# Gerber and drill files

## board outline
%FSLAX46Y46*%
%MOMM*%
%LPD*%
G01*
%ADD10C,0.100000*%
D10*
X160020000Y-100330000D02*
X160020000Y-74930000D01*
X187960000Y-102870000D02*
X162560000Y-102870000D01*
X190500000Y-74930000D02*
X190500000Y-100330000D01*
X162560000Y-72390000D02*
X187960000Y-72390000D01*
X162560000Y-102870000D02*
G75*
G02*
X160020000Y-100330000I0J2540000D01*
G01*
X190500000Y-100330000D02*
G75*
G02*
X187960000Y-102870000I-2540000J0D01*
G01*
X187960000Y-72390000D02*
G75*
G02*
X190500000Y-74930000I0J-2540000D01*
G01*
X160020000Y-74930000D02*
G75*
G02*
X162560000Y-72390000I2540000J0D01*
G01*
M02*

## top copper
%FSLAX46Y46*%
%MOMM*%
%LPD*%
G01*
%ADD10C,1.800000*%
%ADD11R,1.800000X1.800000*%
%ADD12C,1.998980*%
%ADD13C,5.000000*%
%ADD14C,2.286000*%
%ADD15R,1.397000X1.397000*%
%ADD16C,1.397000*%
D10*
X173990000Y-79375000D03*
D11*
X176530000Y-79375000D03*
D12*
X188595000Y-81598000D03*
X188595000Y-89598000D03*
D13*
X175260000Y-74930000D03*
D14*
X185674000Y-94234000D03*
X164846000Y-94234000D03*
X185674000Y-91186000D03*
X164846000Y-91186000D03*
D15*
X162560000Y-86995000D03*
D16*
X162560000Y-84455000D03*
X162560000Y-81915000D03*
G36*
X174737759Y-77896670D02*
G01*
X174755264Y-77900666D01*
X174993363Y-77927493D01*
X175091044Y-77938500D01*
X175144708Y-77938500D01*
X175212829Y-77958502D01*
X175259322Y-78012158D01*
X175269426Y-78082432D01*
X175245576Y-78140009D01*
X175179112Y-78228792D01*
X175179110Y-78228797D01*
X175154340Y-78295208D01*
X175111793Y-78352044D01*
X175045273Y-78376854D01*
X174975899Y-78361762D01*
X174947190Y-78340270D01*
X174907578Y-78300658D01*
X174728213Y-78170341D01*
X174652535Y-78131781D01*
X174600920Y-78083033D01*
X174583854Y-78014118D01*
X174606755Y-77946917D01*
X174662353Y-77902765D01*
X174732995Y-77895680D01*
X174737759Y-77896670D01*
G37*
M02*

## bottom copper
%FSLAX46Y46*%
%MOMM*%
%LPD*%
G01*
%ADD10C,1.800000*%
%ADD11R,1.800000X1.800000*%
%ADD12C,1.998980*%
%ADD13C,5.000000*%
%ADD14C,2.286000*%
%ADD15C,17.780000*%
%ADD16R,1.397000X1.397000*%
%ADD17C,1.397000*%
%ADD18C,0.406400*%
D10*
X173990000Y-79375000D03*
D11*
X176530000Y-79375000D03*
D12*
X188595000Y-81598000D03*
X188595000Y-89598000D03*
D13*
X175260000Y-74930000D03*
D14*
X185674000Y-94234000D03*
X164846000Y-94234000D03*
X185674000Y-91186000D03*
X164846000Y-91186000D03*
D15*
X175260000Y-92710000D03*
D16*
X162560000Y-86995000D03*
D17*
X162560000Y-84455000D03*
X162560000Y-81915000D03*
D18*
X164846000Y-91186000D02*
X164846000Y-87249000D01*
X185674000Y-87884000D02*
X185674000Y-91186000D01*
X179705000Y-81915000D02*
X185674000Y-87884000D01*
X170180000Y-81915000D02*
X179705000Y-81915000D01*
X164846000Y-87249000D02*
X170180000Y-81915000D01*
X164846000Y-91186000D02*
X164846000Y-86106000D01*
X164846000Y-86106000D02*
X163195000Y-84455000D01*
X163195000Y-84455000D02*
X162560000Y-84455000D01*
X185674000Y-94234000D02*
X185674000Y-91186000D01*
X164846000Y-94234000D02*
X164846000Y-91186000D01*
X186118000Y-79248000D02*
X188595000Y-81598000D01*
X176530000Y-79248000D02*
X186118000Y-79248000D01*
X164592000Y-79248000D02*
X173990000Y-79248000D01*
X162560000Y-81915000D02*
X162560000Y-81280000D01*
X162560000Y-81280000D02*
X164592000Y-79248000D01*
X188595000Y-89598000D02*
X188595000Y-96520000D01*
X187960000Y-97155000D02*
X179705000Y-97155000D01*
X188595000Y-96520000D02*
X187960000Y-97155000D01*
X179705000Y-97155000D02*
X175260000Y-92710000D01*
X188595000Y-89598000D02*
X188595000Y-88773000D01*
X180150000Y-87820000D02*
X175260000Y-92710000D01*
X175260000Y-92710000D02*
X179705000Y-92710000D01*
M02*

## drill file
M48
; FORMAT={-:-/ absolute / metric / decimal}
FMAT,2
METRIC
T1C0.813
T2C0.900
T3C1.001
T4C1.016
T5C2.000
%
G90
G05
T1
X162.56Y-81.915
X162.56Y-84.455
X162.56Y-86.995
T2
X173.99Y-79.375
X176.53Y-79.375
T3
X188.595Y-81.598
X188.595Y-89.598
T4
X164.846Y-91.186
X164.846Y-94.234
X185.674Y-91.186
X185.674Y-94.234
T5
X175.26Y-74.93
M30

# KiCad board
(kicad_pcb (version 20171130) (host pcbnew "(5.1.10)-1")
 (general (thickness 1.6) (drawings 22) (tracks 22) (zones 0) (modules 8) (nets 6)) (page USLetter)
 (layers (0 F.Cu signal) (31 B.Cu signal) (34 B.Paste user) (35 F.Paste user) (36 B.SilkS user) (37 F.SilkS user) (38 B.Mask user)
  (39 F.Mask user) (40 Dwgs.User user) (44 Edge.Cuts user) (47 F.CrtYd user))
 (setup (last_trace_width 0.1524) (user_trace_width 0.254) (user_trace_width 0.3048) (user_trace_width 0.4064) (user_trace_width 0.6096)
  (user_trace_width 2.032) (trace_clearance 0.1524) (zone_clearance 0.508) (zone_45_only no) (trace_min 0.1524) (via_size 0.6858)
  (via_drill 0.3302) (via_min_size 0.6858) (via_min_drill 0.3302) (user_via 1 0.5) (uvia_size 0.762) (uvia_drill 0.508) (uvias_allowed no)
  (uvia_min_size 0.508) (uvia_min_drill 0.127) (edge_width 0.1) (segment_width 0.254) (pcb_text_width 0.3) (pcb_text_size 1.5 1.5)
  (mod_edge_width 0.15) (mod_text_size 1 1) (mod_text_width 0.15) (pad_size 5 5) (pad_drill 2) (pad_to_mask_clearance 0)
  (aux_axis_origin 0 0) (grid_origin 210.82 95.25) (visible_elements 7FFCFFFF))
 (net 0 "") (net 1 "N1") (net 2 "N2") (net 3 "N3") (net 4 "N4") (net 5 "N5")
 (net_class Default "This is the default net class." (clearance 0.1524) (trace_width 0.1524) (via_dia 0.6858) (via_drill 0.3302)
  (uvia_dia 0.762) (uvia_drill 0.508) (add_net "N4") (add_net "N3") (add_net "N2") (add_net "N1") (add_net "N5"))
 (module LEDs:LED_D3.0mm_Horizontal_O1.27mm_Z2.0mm (layer F.Cu) (at 173.99 79.375)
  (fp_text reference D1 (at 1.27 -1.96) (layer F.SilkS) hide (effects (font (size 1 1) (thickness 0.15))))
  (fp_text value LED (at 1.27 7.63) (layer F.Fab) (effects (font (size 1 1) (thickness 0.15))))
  (pad 2 thru_hole circle (at 0 0) (size 1.8 1.8) (drill 0.9) (layers *.Cu *.Mask) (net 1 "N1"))
  (pad 1 thru_hole rect (at 2.54 0) (size 1.8 1.8) (drill 0.9) (layers *.Cu *.Mask) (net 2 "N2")))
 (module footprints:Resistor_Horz (layer F.Cu) (at 188.595 85.598 270)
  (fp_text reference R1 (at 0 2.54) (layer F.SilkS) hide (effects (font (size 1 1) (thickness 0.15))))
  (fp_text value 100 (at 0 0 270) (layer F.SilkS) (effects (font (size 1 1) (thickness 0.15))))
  (pad 1 thru_hole circle (at -4 0 270) (size 1.99898 1.99898) (drill 1.00076) (layers *.Cu *.SilkS *.Mask) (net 2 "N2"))
  (pad 2 thru_hole circle (at 4 0 270) (size 1.99898 1.99898) (drill 1.00076) (layers *.Cu *.SilkS *.Mask) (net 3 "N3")))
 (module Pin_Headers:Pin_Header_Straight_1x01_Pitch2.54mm (layer F.Cu) (at 175.26 74.93)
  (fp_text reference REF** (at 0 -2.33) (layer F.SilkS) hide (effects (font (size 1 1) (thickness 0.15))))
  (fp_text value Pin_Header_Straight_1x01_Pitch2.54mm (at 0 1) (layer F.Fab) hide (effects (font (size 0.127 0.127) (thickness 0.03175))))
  (pad 1 thru_hole circle (at 0 0) (size 5 5) (drill 2) (layers *.Cu *.Mask)))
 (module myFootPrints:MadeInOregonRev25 (layer F.Cu) (at 167.64 76.454)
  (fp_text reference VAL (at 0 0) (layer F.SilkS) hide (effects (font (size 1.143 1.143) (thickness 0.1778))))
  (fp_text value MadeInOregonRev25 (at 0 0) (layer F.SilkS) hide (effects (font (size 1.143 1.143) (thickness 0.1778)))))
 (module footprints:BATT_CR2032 (layer B.Cu) (at 175.26 92.71 180)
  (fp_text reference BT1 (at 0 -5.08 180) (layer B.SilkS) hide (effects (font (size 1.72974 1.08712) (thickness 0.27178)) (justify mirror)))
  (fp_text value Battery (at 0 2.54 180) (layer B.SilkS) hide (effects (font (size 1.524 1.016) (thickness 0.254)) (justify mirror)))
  (pad 1 thru_hole circle (at -10.414 -1.524 180) (size 2.286 2.286) (drill 1.016) (layers *.Cu *.Mask B.SilkS) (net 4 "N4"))
  (pad 1 thru_hole circle (at 10.414 -1.524 180) (size 2.286 2.286) (drill 1.016) (layers *.Cu *.Mask B.SilkS) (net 4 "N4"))
  (pad 1 thru_hole circle (at -10.414 1.524 180) (size 2.286 2.286) (drill 1.016) (layers *.Cu *.Mask B.SilkS) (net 4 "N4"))
  (pad 1 thru_hole circle (at 10.414 1.524 180) (size 2.286 2.286) (drill 1.016) (layers *.Cu *.Mask B.SilkS) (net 4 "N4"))
  (pad 2 smd circle (at 0 0 180) (size 17.78 17.78) (layers B.Cu B.Paste B.Mask) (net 3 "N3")))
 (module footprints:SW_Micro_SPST (layer F.Cu) (at 162.56 84.455 90)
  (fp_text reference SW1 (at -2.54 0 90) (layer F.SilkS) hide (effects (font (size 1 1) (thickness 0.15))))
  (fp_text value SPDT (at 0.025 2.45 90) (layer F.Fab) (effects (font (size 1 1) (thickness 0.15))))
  (pad 1 thru_hole rect (at -2.54 0 90) (size 1.397 1.397) (drill 0.8128) (layers *.Cu *.Mask F.SilkS) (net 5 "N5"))
  (pad 2 thru_hole circle (at 0 0 90) (size 1.397 1.397) (drill 0.8128) (layers *.Cu *.Mask F.SilkS) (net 4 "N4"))
  (pad 3 thru_hole circle (at 2.54 0 90) (size 1.397 1.397) (drill 0.8128) (layers *.Cu *.Mask F.SilkS) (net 1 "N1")))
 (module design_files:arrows (layer F.Cu) (at 177.546 81.788)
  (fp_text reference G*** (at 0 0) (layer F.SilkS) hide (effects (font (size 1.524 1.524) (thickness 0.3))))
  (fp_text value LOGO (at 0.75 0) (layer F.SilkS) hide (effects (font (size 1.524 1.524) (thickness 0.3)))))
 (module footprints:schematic (layer F.Cu) (at 175.26 87.503)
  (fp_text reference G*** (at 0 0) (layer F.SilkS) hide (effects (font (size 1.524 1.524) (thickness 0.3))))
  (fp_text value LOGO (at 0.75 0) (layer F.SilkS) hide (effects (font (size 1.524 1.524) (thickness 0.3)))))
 (gr_line (start 160.02 100.33) (end 160.02 74.93) (angle 90) (layer Edge.Cuts) (width 0.1))
 (gr_line (start 187.96 102.87) (end 162.56 102.87) (angle 90) (layer Edge.Cuts) (width 0.1))
 (gr_line (start 190.5 74.93) (end 190.5 100.33) (angle 90) (layer Edge.Cuts) (width 0.1))
 (gr_line (start 162.56 72.39) (end 187.96 72.39) (angle 90) (layer Edge.Cuts) (width 0.1))
 (gr_arc (start 162.56 100.33) (end 162.56 102.87) (angle 90) (layer Edge.Cuts) (width 0.1))
 (gr_arc (start 187.96 100.33) (end 190.5 100.33) (angle 90) (layer Edge.Cuts) (width 0.1))
 (gr_arc (start 187.96 74.93) (end 187.96 72.39) (angle 90) (layer Edge.Cuts) (width 0.1))
 (gr_arc (start 162.56 74.93) (end 160.02 74.93) (angle 90) (layer Edge.Cuts) (width 0.1))
 (segment (start 164.846 91.186) (end 164.846 87.249) (width 0.4064) (layer B.Cu) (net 4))
 (segment (start 185.674 87.884) (end 185.674 91.186) (width 0.4064) (layer B.Cu) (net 4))
 (segment (start 179.705 81.915) (end 185.674 87.884) (width 0.4064) (layer B.Cu) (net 4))
 (segment (start 170.18 81.915) (end 179.705 81.915) (width 0.4064) (layer B.Cu) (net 4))
 (segment (start 164.846 87.249) (end 170.18 81.915) (width 0.4064) (layer B.Cu) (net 4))
 (segment (start 164.846 91.186) (end 164.846 86.106) (width 0.4064) (layer B.Cu) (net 4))
 (segment (start 164.846 86.106) (end 163.195 84.455) (width 0.4064) (layer B.Cu) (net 4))
 (segment (start 163.195 84.455) (end 162.56 84.455) (width 0.4064) (layer B.Cu) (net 4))
 (segment (start 185.674 94.234) (end 185.674 91.186) (width 0.4064) (layer B.Cu) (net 4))
 (segment (start 164.846 94.234) (end 164.846 91.186) (width 0.4064) (layer B.Cu) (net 4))
 (segment (start 186.118 79.248) (end 188.595 81.598) (width 0.4064) (layer B.Cu) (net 2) (status 20))
 (segment (start 176.53 79.248) (end 186.118 79.248) (width 0.4064) (layer B.Cu) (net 2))
 (segment (start 164.592 79.248) (end 173.99 79.248) (width 0.4064) (layer B.Cu) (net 1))
 (segment (start 162.56 81.915) (end 162.56 81.28) (width 0.4064) (layer B.Cu) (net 1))
 (segment (start 162.56 81.28) (end 164.592 79.248) (width 0.4064) (layer B.Cu) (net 1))
 (segment (start 188.595 89.598) (end 188.595 96.52) (width 0.4064) (layer B.Cu) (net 3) (status 10))
 (segment (start 187.96 97.155) (end 179.705 97.155) (width 0.4064) (layer B.Cu) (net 3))
 (segment (start 188.595 96.52) (end 187.96 97.155) (width 0.4064) (layer B.Cu) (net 3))
 (segment (start 179.705 97.155) (end 175.26 92.71) (width 0.4064) (layer B.Cu) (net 3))
 (segment (start 188.595 89.598) (end 188.595 88.773) (width 0.4064) (layer B.Cu) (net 3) (status 30))
 (segment (start 180.15 87.82) (end 175.26 92.71) (width 0.4064) (layer B.Cu) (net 3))
 (segment (start 175.26 92.71) (end 179.705 92.71) (width 0.4064) (layer B.Cu) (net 3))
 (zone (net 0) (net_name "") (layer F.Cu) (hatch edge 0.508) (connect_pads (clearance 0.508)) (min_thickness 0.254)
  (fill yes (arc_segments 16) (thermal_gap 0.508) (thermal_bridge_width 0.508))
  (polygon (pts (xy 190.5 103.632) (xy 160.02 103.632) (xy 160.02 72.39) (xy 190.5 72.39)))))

